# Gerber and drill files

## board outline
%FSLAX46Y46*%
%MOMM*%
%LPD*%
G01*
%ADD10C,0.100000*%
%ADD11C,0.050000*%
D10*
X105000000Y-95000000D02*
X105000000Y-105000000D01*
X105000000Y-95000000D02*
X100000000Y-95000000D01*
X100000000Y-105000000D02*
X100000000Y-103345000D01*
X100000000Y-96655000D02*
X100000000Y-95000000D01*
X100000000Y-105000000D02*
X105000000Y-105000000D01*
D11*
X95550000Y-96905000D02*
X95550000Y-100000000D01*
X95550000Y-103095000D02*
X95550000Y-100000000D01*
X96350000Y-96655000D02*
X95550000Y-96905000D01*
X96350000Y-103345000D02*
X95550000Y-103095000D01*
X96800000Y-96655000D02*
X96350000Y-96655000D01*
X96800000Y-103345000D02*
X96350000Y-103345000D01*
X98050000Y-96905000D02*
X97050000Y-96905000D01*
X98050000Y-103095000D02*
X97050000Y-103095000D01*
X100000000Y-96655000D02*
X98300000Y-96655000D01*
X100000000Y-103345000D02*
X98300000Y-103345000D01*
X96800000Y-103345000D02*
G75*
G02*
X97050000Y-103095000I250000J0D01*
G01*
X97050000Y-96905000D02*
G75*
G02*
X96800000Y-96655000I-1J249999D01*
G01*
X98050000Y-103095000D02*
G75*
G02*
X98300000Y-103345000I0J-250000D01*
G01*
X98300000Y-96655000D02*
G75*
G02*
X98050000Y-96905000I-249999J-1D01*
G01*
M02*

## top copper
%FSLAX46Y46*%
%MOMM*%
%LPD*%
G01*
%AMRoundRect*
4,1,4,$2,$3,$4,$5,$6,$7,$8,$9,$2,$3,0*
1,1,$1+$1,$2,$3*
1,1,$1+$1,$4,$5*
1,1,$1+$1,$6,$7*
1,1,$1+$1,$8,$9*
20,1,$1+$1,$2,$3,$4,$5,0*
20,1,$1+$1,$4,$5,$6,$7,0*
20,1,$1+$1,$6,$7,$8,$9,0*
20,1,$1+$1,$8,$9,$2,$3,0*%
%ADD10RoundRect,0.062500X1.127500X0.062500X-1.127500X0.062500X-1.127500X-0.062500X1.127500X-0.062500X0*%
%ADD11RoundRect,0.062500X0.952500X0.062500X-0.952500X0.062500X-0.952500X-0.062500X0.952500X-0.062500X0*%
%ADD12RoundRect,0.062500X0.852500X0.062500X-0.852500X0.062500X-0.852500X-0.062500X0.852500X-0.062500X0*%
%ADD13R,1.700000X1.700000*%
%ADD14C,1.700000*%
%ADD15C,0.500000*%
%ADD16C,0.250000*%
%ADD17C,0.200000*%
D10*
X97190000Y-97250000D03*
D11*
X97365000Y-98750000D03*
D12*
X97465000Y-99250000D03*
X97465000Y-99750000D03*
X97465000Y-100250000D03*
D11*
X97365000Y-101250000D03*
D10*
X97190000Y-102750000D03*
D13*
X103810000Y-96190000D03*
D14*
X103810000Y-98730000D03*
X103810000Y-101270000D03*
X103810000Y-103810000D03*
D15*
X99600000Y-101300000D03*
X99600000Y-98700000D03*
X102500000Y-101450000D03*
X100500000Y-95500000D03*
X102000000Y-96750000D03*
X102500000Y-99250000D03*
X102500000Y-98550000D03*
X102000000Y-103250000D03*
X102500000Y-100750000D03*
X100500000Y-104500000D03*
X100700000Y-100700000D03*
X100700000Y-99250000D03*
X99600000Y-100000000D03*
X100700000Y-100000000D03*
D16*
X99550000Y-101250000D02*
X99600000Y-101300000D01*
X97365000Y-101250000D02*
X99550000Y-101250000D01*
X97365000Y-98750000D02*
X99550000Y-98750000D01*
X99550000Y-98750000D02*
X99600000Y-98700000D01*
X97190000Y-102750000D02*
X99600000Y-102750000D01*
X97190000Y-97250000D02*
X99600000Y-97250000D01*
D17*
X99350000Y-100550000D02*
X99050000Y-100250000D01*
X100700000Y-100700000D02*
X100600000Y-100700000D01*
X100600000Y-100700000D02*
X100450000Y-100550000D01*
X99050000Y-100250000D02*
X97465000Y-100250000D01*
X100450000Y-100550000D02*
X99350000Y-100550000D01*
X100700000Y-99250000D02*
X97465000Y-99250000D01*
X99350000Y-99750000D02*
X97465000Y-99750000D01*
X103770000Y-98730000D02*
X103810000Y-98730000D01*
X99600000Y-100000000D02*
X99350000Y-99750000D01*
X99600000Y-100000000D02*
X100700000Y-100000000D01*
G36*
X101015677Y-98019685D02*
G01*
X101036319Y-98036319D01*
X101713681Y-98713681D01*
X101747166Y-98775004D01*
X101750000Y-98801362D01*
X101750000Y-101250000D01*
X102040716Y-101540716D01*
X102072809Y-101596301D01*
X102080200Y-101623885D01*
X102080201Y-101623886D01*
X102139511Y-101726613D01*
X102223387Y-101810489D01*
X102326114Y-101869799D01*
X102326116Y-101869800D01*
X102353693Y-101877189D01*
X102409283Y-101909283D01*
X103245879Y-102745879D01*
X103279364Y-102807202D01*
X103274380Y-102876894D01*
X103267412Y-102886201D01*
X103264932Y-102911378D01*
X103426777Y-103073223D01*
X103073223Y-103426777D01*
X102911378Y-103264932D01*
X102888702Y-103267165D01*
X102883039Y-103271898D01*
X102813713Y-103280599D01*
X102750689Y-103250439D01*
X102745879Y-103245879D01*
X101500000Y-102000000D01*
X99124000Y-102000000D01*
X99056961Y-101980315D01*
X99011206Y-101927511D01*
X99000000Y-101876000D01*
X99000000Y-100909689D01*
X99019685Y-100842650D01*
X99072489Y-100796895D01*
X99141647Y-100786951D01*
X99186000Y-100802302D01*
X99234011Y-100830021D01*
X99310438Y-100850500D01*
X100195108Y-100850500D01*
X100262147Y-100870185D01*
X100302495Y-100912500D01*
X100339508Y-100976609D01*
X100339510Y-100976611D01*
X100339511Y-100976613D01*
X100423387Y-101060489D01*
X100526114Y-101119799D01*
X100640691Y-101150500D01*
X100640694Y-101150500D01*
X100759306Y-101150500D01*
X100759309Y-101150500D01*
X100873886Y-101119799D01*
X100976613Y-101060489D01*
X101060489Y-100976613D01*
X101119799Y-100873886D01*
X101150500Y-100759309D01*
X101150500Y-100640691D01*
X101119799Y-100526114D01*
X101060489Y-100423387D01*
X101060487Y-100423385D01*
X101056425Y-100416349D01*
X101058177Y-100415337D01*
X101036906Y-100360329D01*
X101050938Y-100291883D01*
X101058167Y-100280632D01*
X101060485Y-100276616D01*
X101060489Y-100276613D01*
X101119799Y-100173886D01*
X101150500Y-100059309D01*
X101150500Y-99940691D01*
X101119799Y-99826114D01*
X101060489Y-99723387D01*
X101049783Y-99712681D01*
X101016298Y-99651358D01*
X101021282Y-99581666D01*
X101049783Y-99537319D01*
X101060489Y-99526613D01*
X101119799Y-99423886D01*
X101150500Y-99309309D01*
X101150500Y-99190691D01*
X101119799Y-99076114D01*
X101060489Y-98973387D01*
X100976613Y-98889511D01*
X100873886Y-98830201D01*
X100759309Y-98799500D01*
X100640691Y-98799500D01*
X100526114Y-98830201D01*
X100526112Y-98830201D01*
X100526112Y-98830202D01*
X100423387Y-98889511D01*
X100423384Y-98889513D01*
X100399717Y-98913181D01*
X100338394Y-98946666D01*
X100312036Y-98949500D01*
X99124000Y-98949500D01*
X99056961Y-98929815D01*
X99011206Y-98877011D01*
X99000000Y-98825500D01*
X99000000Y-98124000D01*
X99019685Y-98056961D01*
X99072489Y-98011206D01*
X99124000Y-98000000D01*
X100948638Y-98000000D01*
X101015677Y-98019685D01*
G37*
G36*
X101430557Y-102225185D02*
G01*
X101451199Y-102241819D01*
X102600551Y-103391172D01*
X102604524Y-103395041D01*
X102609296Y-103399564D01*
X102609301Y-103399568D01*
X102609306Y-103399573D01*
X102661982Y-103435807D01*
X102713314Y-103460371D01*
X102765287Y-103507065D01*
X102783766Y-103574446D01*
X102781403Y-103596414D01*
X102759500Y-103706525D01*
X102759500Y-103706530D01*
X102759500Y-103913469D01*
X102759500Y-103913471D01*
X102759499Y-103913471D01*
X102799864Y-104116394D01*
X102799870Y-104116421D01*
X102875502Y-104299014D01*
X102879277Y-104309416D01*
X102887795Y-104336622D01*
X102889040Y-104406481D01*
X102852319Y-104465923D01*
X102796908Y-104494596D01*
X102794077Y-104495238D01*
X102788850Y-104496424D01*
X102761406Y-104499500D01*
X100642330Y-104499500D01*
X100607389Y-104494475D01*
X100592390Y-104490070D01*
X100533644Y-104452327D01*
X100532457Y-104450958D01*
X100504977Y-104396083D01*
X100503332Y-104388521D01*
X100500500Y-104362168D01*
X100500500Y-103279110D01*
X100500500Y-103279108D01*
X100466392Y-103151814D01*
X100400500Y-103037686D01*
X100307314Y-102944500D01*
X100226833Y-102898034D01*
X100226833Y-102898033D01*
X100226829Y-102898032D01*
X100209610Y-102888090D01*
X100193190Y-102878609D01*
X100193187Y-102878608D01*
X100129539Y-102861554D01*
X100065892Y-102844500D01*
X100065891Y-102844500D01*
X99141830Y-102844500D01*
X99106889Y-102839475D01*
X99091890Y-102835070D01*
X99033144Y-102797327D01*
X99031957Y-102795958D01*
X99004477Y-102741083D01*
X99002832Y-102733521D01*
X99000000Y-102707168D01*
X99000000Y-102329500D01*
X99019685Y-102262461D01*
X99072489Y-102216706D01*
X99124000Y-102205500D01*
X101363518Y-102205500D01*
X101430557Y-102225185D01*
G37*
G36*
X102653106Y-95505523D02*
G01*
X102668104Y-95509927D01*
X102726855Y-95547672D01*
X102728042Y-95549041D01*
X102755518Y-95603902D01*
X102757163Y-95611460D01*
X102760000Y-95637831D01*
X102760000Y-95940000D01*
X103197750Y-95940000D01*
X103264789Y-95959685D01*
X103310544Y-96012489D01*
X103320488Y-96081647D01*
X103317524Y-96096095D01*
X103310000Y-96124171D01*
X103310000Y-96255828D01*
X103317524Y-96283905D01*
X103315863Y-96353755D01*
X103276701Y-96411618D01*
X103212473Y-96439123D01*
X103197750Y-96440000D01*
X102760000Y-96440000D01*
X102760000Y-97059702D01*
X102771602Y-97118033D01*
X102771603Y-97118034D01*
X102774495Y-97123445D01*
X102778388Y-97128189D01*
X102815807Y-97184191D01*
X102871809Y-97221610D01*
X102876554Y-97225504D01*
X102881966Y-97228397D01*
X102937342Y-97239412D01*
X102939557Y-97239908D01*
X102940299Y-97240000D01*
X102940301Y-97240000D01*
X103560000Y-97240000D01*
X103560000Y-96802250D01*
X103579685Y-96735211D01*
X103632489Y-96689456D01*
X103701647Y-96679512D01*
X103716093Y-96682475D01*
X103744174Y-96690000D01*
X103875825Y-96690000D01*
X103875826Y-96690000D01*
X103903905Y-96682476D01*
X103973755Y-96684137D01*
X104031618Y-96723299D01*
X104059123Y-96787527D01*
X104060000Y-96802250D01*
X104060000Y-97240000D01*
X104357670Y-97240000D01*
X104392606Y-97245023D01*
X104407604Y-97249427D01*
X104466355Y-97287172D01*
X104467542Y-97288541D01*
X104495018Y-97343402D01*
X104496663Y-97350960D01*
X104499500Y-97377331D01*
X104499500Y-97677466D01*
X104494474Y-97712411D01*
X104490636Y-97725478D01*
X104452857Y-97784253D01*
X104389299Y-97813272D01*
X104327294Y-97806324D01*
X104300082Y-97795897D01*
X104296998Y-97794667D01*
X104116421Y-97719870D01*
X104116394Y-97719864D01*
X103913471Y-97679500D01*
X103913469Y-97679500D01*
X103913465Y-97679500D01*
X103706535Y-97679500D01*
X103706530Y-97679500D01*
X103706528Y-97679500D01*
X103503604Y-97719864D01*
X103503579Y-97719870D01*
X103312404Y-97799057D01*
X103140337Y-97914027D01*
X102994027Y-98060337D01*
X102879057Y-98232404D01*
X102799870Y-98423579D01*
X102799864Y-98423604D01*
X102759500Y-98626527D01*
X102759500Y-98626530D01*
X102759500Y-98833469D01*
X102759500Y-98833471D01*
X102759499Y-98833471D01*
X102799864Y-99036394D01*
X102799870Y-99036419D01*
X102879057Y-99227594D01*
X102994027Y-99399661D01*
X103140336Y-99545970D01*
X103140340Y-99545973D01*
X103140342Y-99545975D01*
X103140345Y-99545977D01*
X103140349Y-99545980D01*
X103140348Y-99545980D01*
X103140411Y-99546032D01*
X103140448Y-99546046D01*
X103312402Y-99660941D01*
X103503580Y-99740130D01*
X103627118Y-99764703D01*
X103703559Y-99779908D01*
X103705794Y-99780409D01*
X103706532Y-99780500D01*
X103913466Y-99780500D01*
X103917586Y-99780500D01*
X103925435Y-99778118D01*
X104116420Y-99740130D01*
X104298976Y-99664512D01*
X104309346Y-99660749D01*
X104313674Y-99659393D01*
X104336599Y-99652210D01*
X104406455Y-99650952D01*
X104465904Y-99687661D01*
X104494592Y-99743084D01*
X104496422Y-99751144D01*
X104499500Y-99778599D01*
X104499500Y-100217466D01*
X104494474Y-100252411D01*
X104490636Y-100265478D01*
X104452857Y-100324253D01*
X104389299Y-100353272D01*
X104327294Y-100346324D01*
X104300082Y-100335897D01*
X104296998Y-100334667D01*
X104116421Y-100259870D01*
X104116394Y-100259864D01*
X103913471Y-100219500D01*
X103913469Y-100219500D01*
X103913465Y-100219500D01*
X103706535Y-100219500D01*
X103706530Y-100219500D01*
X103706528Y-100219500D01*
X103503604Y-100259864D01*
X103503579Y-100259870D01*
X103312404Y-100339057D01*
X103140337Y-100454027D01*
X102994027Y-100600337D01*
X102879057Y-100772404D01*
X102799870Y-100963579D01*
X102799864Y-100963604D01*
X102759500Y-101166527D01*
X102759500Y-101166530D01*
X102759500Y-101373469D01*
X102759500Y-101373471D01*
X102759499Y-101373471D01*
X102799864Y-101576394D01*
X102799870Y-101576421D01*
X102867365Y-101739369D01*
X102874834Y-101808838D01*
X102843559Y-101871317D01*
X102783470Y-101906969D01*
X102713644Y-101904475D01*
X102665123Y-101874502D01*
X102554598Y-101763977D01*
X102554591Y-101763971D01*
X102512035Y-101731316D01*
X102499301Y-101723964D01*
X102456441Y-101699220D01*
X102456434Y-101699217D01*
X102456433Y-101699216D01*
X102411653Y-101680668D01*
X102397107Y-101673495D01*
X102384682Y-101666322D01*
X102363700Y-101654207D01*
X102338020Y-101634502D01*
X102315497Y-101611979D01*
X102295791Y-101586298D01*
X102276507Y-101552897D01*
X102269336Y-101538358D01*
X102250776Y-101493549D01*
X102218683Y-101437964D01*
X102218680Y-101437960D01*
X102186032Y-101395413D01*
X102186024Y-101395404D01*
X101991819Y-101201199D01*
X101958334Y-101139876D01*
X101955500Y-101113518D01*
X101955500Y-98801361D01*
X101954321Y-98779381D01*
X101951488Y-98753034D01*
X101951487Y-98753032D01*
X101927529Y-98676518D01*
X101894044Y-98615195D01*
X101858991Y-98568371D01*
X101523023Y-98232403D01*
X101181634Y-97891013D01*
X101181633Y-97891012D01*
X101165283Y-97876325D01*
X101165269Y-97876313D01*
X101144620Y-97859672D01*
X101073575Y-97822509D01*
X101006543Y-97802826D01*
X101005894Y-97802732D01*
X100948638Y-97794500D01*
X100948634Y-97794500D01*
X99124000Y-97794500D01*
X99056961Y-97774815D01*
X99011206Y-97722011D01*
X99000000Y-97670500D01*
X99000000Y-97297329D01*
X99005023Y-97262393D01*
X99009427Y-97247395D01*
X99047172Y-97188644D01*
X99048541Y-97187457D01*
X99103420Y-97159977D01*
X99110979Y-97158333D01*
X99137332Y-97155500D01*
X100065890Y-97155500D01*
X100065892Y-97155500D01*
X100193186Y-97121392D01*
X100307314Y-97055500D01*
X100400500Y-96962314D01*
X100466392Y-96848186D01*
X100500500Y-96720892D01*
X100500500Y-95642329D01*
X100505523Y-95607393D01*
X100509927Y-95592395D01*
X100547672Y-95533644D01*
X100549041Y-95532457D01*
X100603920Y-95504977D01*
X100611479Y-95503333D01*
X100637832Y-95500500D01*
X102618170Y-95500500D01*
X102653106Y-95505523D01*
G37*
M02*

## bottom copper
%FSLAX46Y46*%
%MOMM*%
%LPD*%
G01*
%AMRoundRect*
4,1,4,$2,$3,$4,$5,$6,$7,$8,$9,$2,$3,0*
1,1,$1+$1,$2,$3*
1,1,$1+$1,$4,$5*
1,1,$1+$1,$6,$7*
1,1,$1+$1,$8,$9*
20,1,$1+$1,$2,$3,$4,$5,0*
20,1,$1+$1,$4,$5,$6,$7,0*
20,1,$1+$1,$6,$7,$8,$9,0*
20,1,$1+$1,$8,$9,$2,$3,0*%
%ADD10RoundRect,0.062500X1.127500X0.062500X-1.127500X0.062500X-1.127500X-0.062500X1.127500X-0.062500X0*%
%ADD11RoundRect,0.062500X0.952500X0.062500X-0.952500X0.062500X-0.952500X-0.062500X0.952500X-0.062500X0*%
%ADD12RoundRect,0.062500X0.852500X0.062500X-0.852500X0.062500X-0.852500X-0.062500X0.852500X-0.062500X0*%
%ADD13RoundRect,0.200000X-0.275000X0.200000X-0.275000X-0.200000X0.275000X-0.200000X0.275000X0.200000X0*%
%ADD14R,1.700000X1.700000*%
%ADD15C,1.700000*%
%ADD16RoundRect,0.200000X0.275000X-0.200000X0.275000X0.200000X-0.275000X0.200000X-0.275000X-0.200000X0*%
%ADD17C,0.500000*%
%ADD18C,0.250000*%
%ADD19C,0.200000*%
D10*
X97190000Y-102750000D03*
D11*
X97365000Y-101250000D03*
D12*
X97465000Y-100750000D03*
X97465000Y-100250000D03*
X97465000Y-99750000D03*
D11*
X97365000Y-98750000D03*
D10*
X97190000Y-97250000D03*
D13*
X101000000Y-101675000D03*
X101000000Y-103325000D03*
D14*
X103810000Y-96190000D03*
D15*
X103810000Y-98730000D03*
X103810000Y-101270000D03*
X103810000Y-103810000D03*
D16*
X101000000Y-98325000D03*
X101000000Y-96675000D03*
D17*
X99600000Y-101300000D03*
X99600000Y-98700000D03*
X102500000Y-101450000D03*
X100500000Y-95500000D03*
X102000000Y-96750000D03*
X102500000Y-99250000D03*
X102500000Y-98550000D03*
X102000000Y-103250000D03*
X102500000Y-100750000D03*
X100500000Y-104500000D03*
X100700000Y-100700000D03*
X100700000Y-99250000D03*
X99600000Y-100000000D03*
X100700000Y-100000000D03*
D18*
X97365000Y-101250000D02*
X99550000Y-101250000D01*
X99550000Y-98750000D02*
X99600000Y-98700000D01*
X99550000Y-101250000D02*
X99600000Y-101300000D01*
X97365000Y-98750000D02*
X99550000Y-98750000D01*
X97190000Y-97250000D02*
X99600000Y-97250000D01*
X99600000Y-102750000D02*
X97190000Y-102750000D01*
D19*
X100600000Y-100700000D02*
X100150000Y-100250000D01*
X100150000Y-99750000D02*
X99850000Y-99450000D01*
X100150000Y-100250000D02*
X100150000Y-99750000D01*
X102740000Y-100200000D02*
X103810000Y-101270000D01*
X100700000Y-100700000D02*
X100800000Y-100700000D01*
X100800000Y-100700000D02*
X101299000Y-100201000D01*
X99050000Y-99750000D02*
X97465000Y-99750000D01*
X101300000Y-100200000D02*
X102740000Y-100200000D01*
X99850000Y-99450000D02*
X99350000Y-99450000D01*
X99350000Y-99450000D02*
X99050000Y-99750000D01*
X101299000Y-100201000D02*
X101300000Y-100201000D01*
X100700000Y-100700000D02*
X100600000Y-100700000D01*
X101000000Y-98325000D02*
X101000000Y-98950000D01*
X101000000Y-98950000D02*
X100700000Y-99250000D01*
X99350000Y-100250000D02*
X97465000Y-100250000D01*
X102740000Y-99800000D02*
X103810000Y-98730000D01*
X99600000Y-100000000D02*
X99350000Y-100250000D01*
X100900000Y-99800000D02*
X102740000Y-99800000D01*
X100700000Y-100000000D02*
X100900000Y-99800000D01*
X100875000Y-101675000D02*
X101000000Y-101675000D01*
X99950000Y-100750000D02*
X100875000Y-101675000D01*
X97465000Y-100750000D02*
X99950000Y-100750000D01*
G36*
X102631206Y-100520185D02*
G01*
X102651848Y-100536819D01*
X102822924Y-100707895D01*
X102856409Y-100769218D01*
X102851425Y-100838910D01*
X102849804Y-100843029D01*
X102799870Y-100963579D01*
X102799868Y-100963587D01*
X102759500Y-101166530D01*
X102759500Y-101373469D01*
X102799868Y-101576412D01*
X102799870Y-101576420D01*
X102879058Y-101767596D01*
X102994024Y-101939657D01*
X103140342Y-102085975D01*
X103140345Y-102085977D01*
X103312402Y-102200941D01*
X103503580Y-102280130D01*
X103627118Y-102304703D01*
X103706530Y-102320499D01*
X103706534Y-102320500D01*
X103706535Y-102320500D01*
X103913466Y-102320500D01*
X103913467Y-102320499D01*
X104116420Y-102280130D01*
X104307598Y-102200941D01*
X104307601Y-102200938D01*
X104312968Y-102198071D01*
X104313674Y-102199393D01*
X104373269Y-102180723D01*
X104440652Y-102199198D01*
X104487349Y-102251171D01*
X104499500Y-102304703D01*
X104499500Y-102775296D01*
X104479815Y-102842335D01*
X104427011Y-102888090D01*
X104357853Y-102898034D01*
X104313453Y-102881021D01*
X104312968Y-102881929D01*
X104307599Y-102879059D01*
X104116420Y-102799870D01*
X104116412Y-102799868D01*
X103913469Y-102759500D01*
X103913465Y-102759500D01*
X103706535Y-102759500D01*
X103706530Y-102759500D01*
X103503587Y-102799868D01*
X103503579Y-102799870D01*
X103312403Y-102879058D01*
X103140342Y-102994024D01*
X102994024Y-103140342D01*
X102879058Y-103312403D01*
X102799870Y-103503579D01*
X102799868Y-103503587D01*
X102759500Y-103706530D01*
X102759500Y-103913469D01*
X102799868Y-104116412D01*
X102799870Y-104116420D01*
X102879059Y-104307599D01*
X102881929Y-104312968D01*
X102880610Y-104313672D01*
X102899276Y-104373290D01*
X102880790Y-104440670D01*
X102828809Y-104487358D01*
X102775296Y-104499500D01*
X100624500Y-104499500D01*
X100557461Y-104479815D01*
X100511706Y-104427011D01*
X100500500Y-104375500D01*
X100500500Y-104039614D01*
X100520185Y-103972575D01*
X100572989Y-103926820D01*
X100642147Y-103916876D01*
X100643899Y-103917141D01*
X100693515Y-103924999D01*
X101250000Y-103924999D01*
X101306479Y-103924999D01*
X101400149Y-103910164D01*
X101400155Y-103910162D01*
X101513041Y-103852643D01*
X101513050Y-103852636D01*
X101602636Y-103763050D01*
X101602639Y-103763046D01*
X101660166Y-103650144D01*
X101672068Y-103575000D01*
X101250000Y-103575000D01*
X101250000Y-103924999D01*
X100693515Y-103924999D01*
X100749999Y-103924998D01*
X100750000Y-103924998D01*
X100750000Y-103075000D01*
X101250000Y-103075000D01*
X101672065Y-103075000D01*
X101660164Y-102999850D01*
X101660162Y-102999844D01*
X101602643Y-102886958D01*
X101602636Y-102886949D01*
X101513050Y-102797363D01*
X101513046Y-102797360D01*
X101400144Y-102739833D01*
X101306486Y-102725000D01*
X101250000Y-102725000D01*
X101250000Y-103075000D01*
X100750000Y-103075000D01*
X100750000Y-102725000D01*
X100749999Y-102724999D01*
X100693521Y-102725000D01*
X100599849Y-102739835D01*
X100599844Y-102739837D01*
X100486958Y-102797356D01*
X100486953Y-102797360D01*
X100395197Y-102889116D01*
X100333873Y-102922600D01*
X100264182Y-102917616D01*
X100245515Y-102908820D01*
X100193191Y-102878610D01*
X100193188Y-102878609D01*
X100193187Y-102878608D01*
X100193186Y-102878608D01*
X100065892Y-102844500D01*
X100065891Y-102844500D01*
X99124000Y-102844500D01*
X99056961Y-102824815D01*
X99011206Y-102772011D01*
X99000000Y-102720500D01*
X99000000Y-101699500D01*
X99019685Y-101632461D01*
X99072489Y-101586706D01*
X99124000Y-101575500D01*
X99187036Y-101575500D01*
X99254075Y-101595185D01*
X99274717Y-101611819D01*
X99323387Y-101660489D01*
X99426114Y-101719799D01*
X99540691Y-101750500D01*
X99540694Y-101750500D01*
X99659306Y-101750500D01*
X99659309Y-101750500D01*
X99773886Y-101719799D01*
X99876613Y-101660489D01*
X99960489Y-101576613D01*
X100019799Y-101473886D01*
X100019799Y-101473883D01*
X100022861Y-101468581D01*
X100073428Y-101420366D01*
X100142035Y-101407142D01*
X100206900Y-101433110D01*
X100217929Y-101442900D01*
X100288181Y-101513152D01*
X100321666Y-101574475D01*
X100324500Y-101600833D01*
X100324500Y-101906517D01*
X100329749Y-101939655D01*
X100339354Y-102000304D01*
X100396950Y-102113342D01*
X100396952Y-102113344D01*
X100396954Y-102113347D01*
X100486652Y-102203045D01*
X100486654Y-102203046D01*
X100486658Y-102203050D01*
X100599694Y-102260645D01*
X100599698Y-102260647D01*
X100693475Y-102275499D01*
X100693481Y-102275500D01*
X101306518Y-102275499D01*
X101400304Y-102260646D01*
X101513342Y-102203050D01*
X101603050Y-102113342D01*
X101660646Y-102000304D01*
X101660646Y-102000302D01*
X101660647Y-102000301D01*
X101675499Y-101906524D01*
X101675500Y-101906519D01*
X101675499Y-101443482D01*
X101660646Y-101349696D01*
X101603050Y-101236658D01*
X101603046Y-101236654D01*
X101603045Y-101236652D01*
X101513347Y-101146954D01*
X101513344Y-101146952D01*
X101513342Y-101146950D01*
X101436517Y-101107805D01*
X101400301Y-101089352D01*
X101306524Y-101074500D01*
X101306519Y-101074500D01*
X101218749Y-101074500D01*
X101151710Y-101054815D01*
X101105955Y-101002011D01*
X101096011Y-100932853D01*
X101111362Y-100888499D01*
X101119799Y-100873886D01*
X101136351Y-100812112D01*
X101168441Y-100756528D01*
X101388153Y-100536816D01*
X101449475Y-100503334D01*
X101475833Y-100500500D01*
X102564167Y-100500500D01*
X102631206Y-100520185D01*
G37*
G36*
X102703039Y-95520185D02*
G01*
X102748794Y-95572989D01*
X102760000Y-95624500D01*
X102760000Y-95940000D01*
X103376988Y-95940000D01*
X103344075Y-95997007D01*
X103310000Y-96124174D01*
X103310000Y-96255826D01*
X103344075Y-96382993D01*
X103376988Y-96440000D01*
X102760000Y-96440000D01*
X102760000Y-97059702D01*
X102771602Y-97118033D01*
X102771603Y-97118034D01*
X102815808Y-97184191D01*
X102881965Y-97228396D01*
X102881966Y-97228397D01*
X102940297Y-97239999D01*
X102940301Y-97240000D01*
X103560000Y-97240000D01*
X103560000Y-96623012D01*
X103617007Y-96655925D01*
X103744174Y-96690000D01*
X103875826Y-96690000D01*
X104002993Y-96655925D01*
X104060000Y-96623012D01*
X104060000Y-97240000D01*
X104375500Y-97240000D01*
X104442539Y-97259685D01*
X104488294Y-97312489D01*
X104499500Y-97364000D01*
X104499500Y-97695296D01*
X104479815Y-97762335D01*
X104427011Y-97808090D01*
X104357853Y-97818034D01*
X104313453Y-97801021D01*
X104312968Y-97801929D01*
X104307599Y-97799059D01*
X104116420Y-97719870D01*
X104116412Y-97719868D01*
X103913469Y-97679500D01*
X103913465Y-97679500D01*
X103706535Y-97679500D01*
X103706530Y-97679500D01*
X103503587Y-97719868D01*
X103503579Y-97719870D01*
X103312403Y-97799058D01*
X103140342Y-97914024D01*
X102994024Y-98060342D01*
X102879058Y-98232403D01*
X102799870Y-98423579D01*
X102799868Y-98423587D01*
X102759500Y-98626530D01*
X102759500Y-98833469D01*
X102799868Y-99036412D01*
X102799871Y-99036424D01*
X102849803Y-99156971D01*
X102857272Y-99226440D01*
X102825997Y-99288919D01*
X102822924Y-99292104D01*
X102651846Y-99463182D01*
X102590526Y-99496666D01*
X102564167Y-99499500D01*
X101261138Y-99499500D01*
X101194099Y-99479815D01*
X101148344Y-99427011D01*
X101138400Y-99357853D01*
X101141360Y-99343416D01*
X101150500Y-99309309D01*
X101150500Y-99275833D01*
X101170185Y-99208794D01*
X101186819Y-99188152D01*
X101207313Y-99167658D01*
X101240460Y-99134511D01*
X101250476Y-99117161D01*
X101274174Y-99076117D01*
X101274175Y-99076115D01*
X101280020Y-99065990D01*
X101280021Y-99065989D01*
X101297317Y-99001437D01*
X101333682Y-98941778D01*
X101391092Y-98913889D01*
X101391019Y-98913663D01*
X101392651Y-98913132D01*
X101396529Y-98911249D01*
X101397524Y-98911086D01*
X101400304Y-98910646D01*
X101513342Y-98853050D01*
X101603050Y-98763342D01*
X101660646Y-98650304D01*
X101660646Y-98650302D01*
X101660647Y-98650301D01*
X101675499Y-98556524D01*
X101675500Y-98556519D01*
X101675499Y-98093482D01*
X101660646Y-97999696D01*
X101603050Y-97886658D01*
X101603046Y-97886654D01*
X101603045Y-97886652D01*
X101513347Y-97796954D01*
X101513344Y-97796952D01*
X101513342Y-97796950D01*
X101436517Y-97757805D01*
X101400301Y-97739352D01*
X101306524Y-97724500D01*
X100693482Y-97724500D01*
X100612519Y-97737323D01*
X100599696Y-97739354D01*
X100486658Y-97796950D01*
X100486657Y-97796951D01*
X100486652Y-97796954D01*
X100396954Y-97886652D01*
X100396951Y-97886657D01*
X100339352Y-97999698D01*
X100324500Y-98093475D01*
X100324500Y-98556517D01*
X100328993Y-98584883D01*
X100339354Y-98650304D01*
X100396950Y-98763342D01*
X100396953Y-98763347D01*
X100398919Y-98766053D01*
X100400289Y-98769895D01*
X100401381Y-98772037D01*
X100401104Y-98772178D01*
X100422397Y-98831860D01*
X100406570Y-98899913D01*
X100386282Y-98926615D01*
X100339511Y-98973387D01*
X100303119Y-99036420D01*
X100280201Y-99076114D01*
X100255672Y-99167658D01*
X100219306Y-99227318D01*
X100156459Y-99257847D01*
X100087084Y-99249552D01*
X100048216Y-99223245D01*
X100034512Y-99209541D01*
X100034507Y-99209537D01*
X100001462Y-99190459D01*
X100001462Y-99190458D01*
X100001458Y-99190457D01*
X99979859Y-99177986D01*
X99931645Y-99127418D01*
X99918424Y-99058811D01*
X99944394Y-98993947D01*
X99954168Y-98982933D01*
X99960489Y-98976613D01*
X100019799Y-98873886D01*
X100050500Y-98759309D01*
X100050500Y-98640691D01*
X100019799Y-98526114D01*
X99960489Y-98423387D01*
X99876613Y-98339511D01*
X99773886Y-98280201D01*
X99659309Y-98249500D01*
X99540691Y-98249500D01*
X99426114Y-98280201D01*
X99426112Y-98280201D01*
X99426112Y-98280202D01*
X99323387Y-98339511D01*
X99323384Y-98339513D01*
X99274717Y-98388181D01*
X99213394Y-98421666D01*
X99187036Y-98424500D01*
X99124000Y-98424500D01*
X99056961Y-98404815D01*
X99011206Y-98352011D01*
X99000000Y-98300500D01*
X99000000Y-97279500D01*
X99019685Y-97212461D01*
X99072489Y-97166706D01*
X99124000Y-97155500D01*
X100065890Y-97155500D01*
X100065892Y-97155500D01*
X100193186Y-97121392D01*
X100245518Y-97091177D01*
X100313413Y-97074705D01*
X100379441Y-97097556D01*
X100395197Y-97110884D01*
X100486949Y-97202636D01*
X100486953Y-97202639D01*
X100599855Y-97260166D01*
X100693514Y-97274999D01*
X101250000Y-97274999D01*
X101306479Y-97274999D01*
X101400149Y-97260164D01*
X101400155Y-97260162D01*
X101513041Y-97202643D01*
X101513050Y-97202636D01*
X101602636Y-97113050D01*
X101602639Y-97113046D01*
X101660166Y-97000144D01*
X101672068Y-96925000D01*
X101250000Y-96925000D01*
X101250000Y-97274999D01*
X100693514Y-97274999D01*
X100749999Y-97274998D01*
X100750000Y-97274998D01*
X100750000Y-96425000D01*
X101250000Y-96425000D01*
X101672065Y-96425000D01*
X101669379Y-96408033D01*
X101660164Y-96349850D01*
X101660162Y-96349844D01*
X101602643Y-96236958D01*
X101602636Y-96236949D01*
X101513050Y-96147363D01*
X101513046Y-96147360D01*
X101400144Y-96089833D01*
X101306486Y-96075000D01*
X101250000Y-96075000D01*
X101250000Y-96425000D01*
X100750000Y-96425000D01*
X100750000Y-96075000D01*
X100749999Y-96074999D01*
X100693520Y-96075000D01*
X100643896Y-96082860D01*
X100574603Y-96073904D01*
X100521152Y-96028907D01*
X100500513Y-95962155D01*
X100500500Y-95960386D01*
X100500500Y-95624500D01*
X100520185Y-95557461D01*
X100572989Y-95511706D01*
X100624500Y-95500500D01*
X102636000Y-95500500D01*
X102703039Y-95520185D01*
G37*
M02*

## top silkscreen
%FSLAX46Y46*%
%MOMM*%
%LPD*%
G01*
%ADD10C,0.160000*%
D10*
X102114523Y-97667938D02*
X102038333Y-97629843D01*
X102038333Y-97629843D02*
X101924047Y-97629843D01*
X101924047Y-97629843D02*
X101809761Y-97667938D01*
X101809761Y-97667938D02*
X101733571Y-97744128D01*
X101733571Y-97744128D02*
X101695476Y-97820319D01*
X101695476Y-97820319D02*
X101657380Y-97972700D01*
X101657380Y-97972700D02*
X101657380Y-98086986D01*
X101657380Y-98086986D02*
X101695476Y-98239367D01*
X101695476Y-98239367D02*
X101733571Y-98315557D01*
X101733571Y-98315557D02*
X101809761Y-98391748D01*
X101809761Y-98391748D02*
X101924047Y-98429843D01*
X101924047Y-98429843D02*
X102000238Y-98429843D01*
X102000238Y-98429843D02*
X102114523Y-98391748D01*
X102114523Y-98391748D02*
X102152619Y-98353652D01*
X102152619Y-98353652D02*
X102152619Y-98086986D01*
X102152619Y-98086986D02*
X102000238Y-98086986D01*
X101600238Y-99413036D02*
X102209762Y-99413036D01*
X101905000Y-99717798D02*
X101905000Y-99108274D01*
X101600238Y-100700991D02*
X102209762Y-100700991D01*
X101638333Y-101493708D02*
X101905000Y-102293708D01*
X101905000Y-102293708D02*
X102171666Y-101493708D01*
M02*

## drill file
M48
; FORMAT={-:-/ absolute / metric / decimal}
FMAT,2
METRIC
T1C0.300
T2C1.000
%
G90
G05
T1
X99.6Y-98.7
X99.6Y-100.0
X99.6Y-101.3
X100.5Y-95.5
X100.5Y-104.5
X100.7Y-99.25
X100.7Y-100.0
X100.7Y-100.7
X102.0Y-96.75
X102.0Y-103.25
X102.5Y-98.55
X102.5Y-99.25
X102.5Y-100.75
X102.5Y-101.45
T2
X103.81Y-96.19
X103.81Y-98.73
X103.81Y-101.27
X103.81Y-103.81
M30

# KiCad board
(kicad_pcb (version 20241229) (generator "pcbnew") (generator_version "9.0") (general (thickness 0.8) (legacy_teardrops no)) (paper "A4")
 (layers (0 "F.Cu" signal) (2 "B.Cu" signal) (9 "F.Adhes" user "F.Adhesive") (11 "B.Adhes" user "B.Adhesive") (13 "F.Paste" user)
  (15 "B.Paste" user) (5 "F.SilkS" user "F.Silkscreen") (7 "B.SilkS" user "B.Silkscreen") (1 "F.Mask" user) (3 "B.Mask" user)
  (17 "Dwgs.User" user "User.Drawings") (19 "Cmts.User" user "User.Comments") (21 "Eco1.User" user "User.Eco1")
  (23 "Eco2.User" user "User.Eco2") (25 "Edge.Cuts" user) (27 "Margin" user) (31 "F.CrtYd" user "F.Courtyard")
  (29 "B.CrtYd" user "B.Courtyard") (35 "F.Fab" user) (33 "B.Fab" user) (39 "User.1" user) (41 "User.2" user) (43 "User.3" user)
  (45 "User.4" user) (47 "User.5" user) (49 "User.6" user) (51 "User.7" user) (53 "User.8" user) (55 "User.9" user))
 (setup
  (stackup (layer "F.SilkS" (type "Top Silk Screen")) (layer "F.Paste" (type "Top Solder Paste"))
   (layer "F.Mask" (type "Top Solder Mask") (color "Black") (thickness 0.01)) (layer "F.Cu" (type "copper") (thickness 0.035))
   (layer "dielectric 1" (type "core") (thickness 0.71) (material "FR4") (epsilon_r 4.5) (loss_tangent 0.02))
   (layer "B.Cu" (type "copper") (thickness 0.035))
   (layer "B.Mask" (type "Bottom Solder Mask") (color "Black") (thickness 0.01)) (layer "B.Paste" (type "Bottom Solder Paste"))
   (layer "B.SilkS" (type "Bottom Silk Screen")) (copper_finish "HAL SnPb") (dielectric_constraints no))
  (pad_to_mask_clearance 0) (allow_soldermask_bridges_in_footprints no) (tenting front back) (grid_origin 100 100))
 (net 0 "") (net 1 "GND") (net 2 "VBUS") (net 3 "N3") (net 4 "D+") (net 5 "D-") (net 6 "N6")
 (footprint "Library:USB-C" (layer "F.Cu") (at 100 100 -90)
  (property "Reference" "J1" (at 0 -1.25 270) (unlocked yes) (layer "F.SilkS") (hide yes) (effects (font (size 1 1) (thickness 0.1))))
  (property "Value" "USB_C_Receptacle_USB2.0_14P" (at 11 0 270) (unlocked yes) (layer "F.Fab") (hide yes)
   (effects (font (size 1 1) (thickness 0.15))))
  (fp_line (start -3.095 4.45) (end 0 4.45) (stroke (width 0.05) (type default)) (layer "Edge.Cuts"))
  (fp_line (start 3.095 4.45) (end 0 4.45) (stroke (width 0.05) (type default)) (layer "Edge.Cuts"))
  (fp_line (start -3.345 3.65) (end -3.095 4.45) (stroke (width 0.05) (type default)) (layer "Edge.Cuts"))
  (fp_line (start 3.345 3.65) (end 3.095 4.45) (stroke (width 0.05) (type default)) (layer "Edge.Cuts"))
  (fp_line (start -3.345 3.2) (end -3.345 3.65) (stroke (width 0.05) (type default)) (layer "Edge.Cuts"))
  (fp_line (start 3.345 3.2) (end 3.345 3.65) (stroke (width 0.05) (type default)) (layer "Edge.Cuts"))
  (fp_line (start -3.095 1.95) (end -3.095 2.95) (stroke (width 0.05) (type default)) (layer "Edge.Cuts"))
  (fp_line (start 3.095 1.95) (end 3.095 2.95) (stroke (width 0.05) (type default)) (layer "Edge.Cuts"))
  (fp_line (start -3.345 0) (end -3.345 1.7) (stroke (width 0.05) (type default)) (layer "Edge.Cuts"))
  (fp_line (start 3.345 0) (end 3.345 1.7) (stroke (width 0.05) (type default)) (layer "Edge.Cuts"))
  (fp_arc (start 3.345 3.2) (mid 3.168223 3.126777) (end 3.095 2.95) (stroke (width 0.05) (type default)) (layer "Edge.Cuts"))
  (fp_arc (start -3.095 2.95) (mid -3.168223 3.126777) (end -3.345 3.2) (stroke (width 0.05) (type default)) (layer "Edge.Cuts"))
  (fp_arc (start 3.095 1.95) (mid 3.168223 1.773223) (end 3.345 1.7) (stroke (width 0.05) (type default)) (layer "Edge.Cuts"))
  (fp_arc (start -3.345 1.7) (mid -3.168223 1.773223) (end -3.095 1.95) (stroke (width 0.05) (type default)) (layer "Edge.Cuts"))
  (pad "A1" smd roundrect (at -2.75 2.81 180) (size 2.38 0.25) (layers "F.Cu" "F.Mask" "F.Paste") (roundrect_rratio 0.25) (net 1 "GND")
   (thermal_bridge_angle 45))
  (pad "A4" smd roundrect (at -1.25 2.635 180) (size 2.03 0.25) (layers "F.Cu" "F.Mask" "F.Paste") (roundrect_rratio 0.25) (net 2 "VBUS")
   (thermal_bridge_angle 45))
  (pad "A5" smd roundrect (at -0.75 2.535 180) (size 1.83 0.25) (layers "F.Cu" "F.Mask" "F.Paste") (roundrect_rratio 0.25) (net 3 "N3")
   (thermal_bridge_angle 45))
  (pad "A6" smd roundrect (at -0.25 2.535 180) (size 1.83 0.25) (layers "F.Cu" "F.Mask" "F.Paste") (roundrect_rratio 0.25) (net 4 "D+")
   (thermal_bridge_angle 45))
  (pad "A7" smd roundrect (at 0.25 2.535 180) (size 1.83 0.25) (layers "F.Cu" "F.Mask" "F.Paste") (roundrect_rratio 0.25) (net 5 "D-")
   (thermal_bridge_angle 45))
  (pad "A9" smd roundrect (at 1.25 2.635 180) (size 2.03 0.25) (layers "F.Cu" "F.Mask" "F.Paste") (roundrect_rratio 0.25) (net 2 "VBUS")
   (thermal_bridge_angle 45))
  (pad "A12" smd roundrect (at 2.75 2.81 180) (size 2.38 0.25) (layers "F.Cu" "F.Mask" "F.Paste") (roundrect_rratio 0.25) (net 1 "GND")
   (thermal_bridge_angle 45))
  (pad "B1" smd roundrect (at 2.75 2.81 180) (size 2.38 0.25) (layers "B.Cu" "B.Mask" "B.Paste") (roundrect_rratio 0.25) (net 1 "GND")
   (thermal_bridge_angle 45))
  (pad "B4" smd roundrect (at 1.25 2.635 180) (size 2.03 0.25) (layers "B.Cu" "B.Mask" "B.Paste") (roundrect_rratio 0.25) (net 2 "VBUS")
   (thermal_bridge_angle 45))
  (pad "B5" smd roundrect (at 0.75 2.535 180) (size 1.83 0.25) (layers "B.Cu" "B.Mask" "B.Paste") (roundrect_rratio 0.25) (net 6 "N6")
   (thermal_bridge_angle 45))
  (pad "B6" smd roundrect (at 0.25 2.535 180) (size 1.83 0.25) (layers "B.Cu" "B.Mask" "B.Paste") (roundrect_rratio 0.25) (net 4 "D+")
   (thermal_bridge_angle 45))
  (pad "B7" smd roundrect (at -0.25 2.535 180) (size 1.83 0.25) (layers "B.Cu" "B.Mask" "B.Paste") (roundrect_rratio 0.25) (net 5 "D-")
   (thermal_bridge_angle 45))
  (pad "B9" smd roundrect (at -1.25 2.635 180) (size 2.03 0.25) (layers "B.Cu" "B.Mask" "B.Paste") (roundrect_rratio 0.25) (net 2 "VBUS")
   (thermal_bridge_angle 45))
  (pad "B12" smd roundrect (at -2.75 2.81 180) (size 2.38 0.25) (layers "B.Cu" "B.Mask" "B.Paste") (roundrect_rratio 0.25) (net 1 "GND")
   (thermal_bridge_angle 45)))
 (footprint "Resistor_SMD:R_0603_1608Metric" (layer "B.Cu") (at 101 102.5 -90)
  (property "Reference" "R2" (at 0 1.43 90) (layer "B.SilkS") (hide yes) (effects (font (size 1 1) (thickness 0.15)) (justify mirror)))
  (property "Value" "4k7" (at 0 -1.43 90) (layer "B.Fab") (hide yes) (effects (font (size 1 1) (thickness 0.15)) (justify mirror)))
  (pad "1" smd roundrect (at -0.825 0 270) (size 0.8 0.95) (layers "B.Cu" "B.Mask" "B.Paste") (roundrect_rratio 0.25) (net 6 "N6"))
  (pad "2" smd roundrect (at 0.825 0 270) (size 0.8 0.95) (layers "B.Cu" "B.Mask" "B.Paste") (roundrect_rratio 0.25) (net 1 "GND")))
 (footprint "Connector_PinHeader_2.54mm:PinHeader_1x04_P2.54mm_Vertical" (layer "B.Cu") (at 103.81 96.19 180)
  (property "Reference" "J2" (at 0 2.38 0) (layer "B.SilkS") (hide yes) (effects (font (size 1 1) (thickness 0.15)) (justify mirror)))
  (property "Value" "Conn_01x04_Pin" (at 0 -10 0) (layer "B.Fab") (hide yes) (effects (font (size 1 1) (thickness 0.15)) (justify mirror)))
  (pad "1" thru_hole rect (at 0 0 180) (size 1.7 1.7) (drill 1) (layers "*.Cu" "*.Mask") (remove_unused_layers no) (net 1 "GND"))
  (pad "2" thru_hole circle (at 0 -2.54 180) (size 1.7 1.7) (drill 1) (layers "*.Cu" "*.Mask") (remove_unused_layers no) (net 4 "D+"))
  (pad "3" thru_hole circle (at 0 -5.08 180) (size 1.7 1.7) (drill 1) (layers "*.Cu" "*.Mask") (remove_unused_layers no) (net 5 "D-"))
  (pad "4" thru_hole circle (at 0 -7.62 180) (size 1.7 1.7) (drill 1) (layers "*.Cu" "*.Mask") (remove_unused_layers no) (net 2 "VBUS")))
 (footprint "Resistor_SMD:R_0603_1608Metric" (layer "B.Cu") (at 101 97.5 90)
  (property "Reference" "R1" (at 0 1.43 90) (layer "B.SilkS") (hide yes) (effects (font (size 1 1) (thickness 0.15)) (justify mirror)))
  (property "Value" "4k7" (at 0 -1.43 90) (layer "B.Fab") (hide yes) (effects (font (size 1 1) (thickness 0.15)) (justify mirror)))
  (pad "1" smd roundrect (at -0.825 0 90) (size 0.8 0.95) (layers "B.Cu" "B.Mask" "B.Paste") (roundrect_rratio 0.25) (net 3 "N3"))
  (pad "2" smd roundrect (at 0.825 0 90) (size 0.8 0.95) (layers "B.Cu" "B.Mask" "B.Paste") (roundrect_rratio 0.25) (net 1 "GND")))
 (gr_line (start 105 95) (end 105 105) (stroke (width 0.1) (type default)) (layer "Edge.Cuts"))
 (gr_line (start 105 95) (end 100 95) (stroke (width 0.1) (type default)) (layer "Edge.Cuts"))
 (gr_line (start 100 105) (end 100 103.345) (stroke (width 0.1) (type default)) (layer "Edge.Cuts"))
 (gr_line (start 100 96.655) (end 100 95) (stroke (width 0.1) (type default)) (layer "Edge.Cuts"))
 (gr_line (start 100 105) (end 105 105) (stroke (width 0.1) (type default)) (layer "Edge.Cuts"))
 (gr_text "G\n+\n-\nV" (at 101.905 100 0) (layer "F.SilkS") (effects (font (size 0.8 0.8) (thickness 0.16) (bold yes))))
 (segment (start 99.55 101.25) (end 99.6 101.3) (width 0.25) (layer "F.Cu") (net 2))
 (segment (start 97.365 101.25) (end 99.55 101.25) (width 0.25) (layer "F.Cu") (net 2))
 (segment (start 97.365 98.75) (end 99.55 98.75) (width 0.25) (layer "F.Cu") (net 2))
 (segment (start 99.55 98.75) (end 99.6 98.7) (width 0.25) (layer "F.Cu") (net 2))
 (via (at 99.6 101.3) (size 0.5) (drill 0.3) (layers "F.Cu" "B.Cu") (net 2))
 (via (at 99.6 98.7) (size 0.5) (drill 0.3) (layers "F.Cu" "B.Cu") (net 2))
 (segment (start 97.365 101.25) (end 99.55 101.25) (width 0.25) (layer "B.Cu") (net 2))
 (segment (start 99.55 98.75) (end 99.6 98.7) (width 0.25) (layer "B.Cu") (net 2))
 (segment (start 99.55 101.25) (end 99.6 101.3) (width 0.25) (layer "B.Cu") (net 2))
 (segment (start 97.365 98.75) (end 99.55 98.75) (width 0.25) (layer "B.Cu") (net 2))
 (segment (start 97.19 102.75) (end 99.6 102.75) (width 0.25) (layer "F.Cu") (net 1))
 (segment (start 97.19 97.25) (end 99.6 97.25) (width 0.25) (layer "F.Cu") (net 1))
 (via (at 102.5 101.45) (size 0.5) (drill 0.3) (layers "F.Cu" "B.Cu") (free yes) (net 1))
 (via (at 100.5 95.5) (size 0.5) (drill 0.3) (layers "F.Cu" "B.Cu") (free yes) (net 1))
 (via (at 102 96.75) (size 0.5) (drill 0.3) (layers "F.Cu" "B.Cu") (free yes) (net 1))
 (via (at 102.5 99.25) (size 0.5) (drill 0.3) (layers "F.Cu" "B.Cu") (free yes) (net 1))
 (via (at 102.5 98.55) (size 0.5) (drill 0.3) (layers "F.Cu" "B.Cu") (free yes) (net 1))
 (via (at 102 103.25) (size 0.5) (drill 0.3) (layers "F.Cu" "B.Cu") (free yes) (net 1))
 (via (at 102.5 100.75) (size 0.5) (drill 0.3) (layers "F.Cu" "B.Cu") (free yes) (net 1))
 (via (at 100.5 104.5) (size 0.5) (drill 0.3) (layers "F.Cu" "B.Cu") (free yes) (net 1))
 (segment (start 97.19 97.25) (end 99.6 97.25) (width 0.25) (layer "B.Cu") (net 1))
 (segment (start 99.6 102.75) (end 97.19 102.75) (width 0.25) (layer "B.Cu") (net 1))
 (segment (start 99.35 100.55) (end 99.05 100.25) (width 0.2) (layer "F.Cu") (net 5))
 (segment (start 100.7 100.7) (end 100.6 100.7) (width 0.2) (layer "F.Cu") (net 5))
 (segment (start 100.6 100.7) (end 100.45 100.55) (width 0.2) (layer "F.Cu") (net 5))
 (segment (start 99.05 100.25) (end 97.465 100.25) (width 0.2) (layer "F.Cu") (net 5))
 (segment (start 100.45 100.55) (end 99.35 100.55) (width 0.2) (layer "F.Cu") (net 5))
 (via (at 100.7 100.7) (size 0.5) (drill 0.3) (layers "F.Cu" "B.Cu") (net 5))
 (segment (start 100.6 100.7) (end 100.15 100.25) (width 0.2) (layer "B.Cu") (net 5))
 (segment (start 100.15 99.75) (end 99.85 99.45) (width 0.2) (layer "B.Cu") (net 5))
 (segment (start 100.15 100.25) (end 100.15 99.75) (width 0.2) (layer "B.Cu") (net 5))
 (segment (start 102.74 100.2) (end 103.81 101.27) (width 0.2) (layer "B.Cu") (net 5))
 (segment (start 100.7 100.7) (end 100.8 100.7) (width 0.2) (layer "B.Cu") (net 5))
 (segment (start 100.8 100.7) (end 101.299 100.201) (width 0.2) (layer "B.Cu") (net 5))
 (segment (start 99.05 99.75) (end 97.465 99.75) (width 0.2) (layer "B.Cu") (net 5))
 (segment (start 101.3 100.2) (end 102.74 100.2) (width 0.2) (layer "B.Cu") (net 5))
 (segment (start 99.85 99.45) (end 99.35 99.45) (width 0.2) (layer "B.Cu") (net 5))
 (segment (start 99.35 99.45) (end 99.05 99.75) (width 0.2) (layer "B.Cu") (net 5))
 (segment (start 101.299 100.201) (end 101.3 100.201) (width 0.2) (layer "B.Cu") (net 5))
 (segment (start 100.7 100.7) (end 100.6 100.7) (width 0.2) (layer "B.Cu") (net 5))
 (segment (start 100.7 99.25) (end 97.465 99.25) (width 0.2) (layer "F.Cu") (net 3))
 (via (at 100.7 99.25) (size 0.5) (drill 0.3) (layers "F.Cu" "B.Cu") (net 3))
 (segment (start 101 98.325) (end 101 98.95) (width 0.2) (layer "B.Cu") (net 3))
 (segment (start 101 98.95) (end 100.7 99.25) (width 0.2) (layer "B.Cu") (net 3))
 (segment (start 99.35 99.75) (end 97.465 99.75) (width 0.2) (layer "F.Cu") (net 4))
 (segment (start 103.77 98.73) (end 103.81 98.73) (width 0.2) (layer "F.Cu") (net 4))
 (segment (start 99.6 100) (end 99.35 99.75) (width 0.2) (layer "F.Cu") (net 4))
 (segment (start 99.6 100) (end 100.7 100) (width 0.2) (layer "F.Cu") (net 4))
 (via (at 99.6 100) (size 0.5) (drill 0.3) (layers "F.Cu" "B.Cu") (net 4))
 (via (at 100.7 100) (size 0.5) (drill 0.3) (layers "F.Cu" "B.Cu") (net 4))
 (segment (start 99.35 100.25) (end 97.465 100.25) (width 0.2) (layer "B.Cu") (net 4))
 (segment (start 102.74 99.8) (end 103.81 98.73) (width 0.2) (layer "B.Cu") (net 4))
 (segment (start 99.6 100) (end 99.35 100.25) (width 0.2) (layer "B.Cu") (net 4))
 (segment (start 100.9 99.8) (end 102.74 99.8) (width 0.2) (layer "B.Cu") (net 4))
 (segment (start 100.7 100) (end 100.9 99.8) (width 0.2) (layer "B.Cu") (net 4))
 (segment (start 100.875 101.675) (end 101 101.675) (width 0.2) (layer "B.Cu") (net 6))
 (segment (start 99.95 100.75) (end 100.875 101.675) (width 0.2) (layer "B.Cu") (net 6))
 (segment (start 97.465 100.75) (end 99.95 100.75) (width 0.2) (layer "B.Cu") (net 6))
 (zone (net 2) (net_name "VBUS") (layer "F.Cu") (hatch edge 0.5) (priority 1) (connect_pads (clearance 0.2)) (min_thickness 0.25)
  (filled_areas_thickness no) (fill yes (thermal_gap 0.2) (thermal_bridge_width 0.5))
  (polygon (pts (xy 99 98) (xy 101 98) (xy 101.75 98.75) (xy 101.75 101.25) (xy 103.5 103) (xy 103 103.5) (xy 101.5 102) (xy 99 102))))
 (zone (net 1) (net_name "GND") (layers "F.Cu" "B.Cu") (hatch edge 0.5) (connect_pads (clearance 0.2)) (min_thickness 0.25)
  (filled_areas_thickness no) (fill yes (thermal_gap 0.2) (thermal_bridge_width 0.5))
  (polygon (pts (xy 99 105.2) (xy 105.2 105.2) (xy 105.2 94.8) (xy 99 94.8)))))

